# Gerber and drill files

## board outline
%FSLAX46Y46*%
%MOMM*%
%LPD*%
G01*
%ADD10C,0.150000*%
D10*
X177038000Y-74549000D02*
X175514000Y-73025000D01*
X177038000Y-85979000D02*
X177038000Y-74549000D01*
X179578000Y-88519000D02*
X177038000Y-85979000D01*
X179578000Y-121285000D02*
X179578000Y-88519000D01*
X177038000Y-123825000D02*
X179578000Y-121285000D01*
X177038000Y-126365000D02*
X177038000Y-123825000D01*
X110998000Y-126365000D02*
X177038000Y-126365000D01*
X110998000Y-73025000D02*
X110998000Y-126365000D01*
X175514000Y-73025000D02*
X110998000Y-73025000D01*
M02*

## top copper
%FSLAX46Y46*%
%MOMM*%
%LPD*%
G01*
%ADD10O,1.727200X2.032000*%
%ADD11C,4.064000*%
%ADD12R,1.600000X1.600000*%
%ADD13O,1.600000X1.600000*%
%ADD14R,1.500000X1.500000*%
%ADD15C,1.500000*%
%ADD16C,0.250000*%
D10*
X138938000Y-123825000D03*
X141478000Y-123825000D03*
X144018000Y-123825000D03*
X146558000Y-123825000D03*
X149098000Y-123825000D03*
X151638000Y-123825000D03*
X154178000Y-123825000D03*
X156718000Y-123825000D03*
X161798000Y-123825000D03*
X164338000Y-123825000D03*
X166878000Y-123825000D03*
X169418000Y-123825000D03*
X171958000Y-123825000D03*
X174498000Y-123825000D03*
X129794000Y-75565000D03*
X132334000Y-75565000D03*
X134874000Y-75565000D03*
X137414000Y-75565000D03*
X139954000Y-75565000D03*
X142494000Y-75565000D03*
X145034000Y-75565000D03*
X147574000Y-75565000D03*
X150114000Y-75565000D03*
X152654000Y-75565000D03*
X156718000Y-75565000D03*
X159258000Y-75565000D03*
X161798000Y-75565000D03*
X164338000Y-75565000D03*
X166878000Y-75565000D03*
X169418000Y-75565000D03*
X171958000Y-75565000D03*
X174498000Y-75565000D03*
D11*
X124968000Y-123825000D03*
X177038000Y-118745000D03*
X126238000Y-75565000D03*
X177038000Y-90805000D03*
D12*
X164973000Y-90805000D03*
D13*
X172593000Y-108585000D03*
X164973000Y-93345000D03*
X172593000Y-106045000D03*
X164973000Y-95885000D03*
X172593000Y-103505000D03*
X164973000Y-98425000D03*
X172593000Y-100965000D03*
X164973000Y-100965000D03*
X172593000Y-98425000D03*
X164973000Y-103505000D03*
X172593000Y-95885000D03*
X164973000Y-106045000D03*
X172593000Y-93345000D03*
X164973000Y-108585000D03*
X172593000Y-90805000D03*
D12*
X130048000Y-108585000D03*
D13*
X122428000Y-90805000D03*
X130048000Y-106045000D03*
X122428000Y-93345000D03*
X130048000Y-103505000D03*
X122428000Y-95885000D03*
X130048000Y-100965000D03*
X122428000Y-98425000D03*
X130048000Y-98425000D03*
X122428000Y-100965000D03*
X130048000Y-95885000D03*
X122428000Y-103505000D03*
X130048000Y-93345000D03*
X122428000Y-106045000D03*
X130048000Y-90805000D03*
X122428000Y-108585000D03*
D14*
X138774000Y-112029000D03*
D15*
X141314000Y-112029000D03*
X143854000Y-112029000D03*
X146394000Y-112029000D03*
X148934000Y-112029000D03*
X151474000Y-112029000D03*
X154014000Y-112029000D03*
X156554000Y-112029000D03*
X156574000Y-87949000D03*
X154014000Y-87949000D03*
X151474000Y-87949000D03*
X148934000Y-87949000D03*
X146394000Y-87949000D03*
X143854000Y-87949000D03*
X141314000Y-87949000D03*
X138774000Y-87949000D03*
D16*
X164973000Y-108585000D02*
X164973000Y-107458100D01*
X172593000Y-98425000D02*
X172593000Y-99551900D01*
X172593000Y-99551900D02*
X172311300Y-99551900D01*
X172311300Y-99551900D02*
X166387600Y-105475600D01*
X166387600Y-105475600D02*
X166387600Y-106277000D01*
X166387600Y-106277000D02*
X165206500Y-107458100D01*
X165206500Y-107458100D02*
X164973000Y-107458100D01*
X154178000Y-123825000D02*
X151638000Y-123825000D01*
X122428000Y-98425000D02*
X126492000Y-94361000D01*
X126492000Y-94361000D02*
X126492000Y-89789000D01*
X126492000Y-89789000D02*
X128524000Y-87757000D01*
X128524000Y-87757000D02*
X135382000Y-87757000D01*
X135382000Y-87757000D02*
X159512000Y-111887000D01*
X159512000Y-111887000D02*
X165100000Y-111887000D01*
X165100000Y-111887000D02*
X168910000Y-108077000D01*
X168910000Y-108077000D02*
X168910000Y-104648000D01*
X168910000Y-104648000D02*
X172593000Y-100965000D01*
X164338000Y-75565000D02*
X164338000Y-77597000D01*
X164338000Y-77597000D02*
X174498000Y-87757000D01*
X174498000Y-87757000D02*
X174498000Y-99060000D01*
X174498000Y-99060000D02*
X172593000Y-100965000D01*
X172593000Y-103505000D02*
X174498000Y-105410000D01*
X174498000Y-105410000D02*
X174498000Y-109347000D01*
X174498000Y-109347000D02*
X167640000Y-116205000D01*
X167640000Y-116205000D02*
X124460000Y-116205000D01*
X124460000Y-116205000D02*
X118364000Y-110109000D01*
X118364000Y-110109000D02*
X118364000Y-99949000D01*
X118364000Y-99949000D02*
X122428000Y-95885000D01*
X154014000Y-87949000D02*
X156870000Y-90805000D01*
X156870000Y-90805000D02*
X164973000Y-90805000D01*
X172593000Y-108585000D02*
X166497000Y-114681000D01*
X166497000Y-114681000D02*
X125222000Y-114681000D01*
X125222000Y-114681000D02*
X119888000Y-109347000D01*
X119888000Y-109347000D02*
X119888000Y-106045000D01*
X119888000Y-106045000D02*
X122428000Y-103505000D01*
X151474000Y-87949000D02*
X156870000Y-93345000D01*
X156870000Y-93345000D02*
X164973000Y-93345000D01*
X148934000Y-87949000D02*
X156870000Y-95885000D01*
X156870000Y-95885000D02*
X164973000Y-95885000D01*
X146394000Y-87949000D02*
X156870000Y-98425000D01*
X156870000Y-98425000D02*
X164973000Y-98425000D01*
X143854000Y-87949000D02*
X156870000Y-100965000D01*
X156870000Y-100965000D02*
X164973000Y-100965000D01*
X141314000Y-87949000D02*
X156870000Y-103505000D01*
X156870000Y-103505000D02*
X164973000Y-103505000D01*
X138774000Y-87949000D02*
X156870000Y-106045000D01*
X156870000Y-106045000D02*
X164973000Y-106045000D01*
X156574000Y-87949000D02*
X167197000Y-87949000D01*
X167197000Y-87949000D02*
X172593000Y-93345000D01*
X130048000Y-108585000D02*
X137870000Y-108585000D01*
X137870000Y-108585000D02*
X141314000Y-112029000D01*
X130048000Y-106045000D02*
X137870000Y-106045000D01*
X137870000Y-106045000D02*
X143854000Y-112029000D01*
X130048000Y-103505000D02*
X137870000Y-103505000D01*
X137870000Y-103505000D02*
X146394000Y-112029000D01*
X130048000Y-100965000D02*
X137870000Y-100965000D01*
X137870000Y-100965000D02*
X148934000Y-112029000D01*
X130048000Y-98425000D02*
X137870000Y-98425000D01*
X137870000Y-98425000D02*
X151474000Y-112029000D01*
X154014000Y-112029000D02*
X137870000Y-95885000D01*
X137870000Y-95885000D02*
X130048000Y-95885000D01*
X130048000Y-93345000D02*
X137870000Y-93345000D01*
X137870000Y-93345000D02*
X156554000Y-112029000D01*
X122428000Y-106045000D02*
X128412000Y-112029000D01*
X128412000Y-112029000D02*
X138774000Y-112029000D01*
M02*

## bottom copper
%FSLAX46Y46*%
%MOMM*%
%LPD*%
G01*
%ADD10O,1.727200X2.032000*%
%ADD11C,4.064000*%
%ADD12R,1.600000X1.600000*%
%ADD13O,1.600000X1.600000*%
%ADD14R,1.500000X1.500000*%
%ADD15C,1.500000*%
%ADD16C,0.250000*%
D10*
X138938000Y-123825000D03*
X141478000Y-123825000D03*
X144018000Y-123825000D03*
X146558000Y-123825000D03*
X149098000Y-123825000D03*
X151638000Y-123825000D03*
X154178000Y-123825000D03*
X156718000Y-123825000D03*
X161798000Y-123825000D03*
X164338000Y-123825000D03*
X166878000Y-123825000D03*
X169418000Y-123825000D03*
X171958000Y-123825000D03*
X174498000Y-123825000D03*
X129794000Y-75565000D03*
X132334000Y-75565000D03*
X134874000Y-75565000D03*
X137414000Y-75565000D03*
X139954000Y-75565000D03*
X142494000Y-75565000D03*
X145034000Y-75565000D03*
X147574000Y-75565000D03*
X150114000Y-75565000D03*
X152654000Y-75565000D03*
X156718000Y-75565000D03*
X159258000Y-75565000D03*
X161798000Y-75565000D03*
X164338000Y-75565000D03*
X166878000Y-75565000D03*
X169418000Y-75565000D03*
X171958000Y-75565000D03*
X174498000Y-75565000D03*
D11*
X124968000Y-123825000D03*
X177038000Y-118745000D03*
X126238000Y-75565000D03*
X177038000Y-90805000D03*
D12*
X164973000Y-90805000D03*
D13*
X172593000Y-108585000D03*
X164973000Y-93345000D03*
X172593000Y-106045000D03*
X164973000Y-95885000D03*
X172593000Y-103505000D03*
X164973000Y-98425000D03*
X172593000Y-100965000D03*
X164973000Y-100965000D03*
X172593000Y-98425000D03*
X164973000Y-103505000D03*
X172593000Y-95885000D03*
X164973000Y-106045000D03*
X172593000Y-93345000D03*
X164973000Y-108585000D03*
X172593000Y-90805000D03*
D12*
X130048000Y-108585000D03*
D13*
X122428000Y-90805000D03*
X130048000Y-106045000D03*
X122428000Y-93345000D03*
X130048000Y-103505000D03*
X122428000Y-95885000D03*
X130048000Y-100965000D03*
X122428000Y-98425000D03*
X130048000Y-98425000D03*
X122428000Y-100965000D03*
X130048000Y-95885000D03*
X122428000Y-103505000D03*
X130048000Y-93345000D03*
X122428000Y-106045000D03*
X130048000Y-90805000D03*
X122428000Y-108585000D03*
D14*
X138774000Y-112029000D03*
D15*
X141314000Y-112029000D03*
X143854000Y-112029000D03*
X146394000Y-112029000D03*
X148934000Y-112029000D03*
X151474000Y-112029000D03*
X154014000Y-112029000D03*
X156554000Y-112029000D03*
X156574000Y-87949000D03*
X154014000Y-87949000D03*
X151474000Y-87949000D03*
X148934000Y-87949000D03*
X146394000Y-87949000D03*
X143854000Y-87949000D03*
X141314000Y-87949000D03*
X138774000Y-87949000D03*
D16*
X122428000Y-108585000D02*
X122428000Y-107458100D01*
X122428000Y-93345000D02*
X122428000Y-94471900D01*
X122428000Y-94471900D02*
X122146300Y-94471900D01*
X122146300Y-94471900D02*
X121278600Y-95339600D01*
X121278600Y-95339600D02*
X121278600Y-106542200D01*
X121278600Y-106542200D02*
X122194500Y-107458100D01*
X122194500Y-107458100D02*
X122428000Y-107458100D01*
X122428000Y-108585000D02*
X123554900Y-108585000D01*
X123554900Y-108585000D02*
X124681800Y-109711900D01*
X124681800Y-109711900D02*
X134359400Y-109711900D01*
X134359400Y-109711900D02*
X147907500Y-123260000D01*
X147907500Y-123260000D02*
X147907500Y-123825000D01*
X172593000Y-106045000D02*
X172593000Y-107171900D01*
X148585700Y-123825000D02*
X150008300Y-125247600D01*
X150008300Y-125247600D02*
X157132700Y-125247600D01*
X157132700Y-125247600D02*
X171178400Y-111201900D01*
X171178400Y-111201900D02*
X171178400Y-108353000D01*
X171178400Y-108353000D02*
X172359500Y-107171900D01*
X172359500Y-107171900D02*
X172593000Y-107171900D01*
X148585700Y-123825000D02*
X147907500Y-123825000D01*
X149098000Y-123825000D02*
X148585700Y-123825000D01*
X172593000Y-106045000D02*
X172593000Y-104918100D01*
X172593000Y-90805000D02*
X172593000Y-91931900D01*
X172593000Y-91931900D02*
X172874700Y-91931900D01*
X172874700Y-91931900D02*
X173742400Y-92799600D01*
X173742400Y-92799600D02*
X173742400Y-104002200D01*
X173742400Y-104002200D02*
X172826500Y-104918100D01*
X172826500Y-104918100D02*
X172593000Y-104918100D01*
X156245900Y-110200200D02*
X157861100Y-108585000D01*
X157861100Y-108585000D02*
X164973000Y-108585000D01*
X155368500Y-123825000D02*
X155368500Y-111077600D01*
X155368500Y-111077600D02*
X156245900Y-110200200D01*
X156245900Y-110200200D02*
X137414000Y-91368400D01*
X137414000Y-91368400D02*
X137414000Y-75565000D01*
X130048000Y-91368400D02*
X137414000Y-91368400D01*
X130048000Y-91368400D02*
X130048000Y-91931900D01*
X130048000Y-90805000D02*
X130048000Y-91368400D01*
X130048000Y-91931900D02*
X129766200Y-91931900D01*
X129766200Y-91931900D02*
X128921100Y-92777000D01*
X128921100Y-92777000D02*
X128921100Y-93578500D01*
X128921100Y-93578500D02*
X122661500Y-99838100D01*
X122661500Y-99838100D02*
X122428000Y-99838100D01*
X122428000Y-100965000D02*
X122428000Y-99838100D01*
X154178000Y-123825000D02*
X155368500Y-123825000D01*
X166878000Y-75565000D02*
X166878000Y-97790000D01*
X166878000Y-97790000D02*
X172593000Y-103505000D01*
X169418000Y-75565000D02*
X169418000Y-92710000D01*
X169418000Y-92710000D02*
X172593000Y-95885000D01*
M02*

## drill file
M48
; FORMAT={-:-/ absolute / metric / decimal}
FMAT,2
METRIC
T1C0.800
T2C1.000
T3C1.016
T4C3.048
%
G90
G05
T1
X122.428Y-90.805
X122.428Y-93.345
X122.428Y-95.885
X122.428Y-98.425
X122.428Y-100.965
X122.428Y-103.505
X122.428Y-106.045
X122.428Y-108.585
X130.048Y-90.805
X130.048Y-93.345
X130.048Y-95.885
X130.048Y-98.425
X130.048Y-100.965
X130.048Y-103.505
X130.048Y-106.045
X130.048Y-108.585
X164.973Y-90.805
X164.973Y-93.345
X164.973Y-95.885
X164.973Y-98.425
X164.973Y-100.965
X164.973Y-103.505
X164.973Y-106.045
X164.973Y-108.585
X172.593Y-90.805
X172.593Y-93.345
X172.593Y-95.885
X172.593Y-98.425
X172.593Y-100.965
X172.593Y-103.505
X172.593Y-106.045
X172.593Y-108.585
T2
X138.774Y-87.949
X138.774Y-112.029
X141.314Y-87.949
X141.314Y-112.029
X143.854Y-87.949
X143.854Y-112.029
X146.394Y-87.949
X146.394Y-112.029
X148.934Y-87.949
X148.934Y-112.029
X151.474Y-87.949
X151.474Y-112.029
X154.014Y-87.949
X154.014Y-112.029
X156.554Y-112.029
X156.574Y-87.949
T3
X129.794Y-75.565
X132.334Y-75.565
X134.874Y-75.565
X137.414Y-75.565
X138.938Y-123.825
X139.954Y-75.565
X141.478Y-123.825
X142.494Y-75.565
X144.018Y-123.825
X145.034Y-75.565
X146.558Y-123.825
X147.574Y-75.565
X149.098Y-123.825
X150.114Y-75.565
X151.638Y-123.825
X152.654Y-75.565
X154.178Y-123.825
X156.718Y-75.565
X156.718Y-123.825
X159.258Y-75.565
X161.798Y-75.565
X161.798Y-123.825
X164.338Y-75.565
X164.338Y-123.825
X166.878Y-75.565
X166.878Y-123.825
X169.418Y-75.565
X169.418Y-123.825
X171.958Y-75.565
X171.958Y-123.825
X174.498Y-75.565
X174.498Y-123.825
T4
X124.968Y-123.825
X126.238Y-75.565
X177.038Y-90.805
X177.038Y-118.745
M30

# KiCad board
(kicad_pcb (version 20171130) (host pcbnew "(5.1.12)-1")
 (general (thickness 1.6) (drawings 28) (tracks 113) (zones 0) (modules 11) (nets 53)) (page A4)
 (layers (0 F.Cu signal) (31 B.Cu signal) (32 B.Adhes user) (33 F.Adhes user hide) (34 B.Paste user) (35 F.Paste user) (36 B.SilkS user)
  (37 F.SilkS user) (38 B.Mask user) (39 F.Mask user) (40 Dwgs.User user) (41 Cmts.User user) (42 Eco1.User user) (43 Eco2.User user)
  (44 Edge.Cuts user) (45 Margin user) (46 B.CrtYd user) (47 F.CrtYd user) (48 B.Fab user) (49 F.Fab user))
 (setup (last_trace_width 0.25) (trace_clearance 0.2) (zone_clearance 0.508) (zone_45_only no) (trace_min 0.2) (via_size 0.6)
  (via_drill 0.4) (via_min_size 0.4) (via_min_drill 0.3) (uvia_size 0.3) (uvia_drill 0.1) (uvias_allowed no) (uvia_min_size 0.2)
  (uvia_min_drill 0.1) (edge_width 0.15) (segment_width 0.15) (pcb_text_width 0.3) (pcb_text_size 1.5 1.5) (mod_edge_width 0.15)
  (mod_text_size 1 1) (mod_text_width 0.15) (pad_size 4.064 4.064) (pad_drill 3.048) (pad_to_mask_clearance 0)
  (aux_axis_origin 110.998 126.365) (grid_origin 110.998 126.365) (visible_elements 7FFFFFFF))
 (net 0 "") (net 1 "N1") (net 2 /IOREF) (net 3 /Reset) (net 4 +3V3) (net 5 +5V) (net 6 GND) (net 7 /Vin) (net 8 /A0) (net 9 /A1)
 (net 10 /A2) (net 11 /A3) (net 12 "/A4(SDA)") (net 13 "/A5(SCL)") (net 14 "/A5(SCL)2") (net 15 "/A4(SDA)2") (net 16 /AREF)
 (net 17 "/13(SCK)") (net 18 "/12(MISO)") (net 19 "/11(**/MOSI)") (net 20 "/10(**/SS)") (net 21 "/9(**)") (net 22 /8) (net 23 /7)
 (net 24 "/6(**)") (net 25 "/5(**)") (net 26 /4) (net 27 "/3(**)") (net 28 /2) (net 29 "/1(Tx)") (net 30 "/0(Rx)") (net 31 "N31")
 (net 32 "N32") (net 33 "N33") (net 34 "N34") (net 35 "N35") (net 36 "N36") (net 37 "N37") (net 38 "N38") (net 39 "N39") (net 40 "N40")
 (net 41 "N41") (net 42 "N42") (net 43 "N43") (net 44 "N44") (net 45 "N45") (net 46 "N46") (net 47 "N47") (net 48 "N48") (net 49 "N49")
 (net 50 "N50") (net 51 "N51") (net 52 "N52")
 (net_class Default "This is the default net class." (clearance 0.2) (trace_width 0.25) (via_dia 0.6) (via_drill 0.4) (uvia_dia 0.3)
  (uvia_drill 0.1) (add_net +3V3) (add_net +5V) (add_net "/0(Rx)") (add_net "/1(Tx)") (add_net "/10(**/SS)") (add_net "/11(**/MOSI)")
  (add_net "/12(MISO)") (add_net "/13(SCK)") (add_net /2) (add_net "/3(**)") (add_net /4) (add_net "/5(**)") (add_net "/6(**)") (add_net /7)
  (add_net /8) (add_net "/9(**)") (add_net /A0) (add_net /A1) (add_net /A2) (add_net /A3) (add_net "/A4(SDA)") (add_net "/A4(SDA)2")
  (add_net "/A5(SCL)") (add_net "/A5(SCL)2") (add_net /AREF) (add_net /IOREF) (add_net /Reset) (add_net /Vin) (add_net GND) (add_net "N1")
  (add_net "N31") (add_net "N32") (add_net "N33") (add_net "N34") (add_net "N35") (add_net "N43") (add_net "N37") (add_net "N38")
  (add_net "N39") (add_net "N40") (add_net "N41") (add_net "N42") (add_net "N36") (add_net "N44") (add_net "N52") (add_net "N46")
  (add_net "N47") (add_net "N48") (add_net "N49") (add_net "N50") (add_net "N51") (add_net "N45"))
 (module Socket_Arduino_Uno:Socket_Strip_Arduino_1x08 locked (layer F.Cu) (at 138.938 123.825)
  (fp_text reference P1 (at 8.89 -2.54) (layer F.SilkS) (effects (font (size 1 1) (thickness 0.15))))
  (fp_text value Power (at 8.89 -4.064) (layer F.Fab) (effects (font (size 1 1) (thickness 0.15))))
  (pad 1 thru_hole oval (at 0 0) (size 1.7272 2.032) (drill 1.016) (layers *.Cu *.Mask F.SilkS) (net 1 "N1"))
  (pad 2 thru_hole oval (at 2.54 0) (size 1.7272 2.032) (drill 1.016) (layers *.Cu *.Mask F.SilkS) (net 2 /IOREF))
  (pad 3 thru_hole oval (at 5.08 0) (size 1.7272 2.032) (drill 1.016) (layers *.Cu *.Mask F.SilkS) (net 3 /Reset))
  (pad 4 thru_hole oval (at 7.62 0) (size 1.7272 2.032) (drill 1.016) (layers *.Cu *.Mask F.SilkS) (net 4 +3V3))
  (pad 5 thru_hole oval (at 10.16 0) (size 1.7272 2.032) (drill 1.016) (layers *.Cu *.Mask F.SilkS) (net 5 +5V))
  (pad 6 thru_hole oval (at 12.7 0) (size 1.7272 2.032) (drill 1.016) (layers *.Cu *.Mask F.SilkS) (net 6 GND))
  (pad 7 thru_hole oval (at 15.24 0) (size 1.7272 2.032) (drill 1.016) (layers *.Cu *.Mask F.SilkS) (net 6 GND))
  (pad 8 thru_hole oval (at 17.78 0) (size 1.7272 2.032) (drill 1.016) (layers *.Cu *.Mask F.SilkS) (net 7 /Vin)))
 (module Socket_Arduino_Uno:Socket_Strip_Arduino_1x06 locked (layer F.Cu) (at 161.798 123.825)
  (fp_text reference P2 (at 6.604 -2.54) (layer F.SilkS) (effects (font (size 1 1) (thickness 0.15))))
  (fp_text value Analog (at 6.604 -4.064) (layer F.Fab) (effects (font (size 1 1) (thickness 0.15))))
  (pad 1 thru_hole oval (at 0 0) (size 1.7272 2.032) (drill 1.016) (layers *.Cu *.Mask F.SilkS) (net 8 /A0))
  (pad 2 thru_hole oval (at 2.54 0) (size 1.7272 2.032) (drill 1.016) (layers *.Cu *.Mask F.SilkS) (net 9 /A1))
  (pad 3 thru_hole oval (at 5.08 0) (size 1.7272 2.032) (drill 1.016) (layers *.Cu *.Mask F.SilkS) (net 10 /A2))
  (pad 4 thru_hole oval (at 7.62 0) (size 1.7272 2.032) (drill 1.016) (layers *.Cu *.Mask F.SilkS) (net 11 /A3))
  (pad 5 thru_hole oval (at 10.16 0) (size 1.7272 2.032) (drill 1.016) (layers *.Cu *.Mask F.SilkS) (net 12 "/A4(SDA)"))
  (pad 6 thru_hole oval (at 12.7 0) (size 1.7272 2.032) (drill 1.016) (layers *.Cu *.Mask F.SilkS) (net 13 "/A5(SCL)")))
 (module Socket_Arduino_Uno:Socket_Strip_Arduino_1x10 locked (layer F.Cu) (at 129.794 75.565)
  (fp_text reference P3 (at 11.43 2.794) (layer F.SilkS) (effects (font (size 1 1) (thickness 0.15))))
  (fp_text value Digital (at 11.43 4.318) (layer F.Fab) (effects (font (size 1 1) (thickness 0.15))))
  (pad 1 thru_hole oval (at 0 0) (size 1.7272 2.032) (drill 1.016) (layers *.Cu *.Mask F.SilkS) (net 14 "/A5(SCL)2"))
  (pad 2 thru_hole oval (at 2.54 0) (size 1.7272 2.032) (drill 1.016) (layers *.Cu *.Mask F.SilkS) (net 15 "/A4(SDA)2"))
  (pad 3 thru_hole oval (at 5.08 0) (size 1.7272 2.032) (drill 1.016) (layers *.Cu *.Mask F.SilkS) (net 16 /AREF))
  (pad 4 thru_hole oval (at 7.62 0) (size 1.7272 2.032) (drill 1.016) (layers *.Cu *.Mask F.SilkS) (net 6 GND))
  (pad 5 thru_hole oval (at 10.16 0) (size 1.7272 2.032) (drill 1.016) (layers *.Cu *.Mask F.SilkS) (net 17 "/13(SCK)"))
  (pad 6 thru_hole oval (at 12.7 0) (size 1.7272 2.032) (drill 1.016) (layers *.Cu *.Mask F.SilkS) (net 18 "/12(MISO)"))
  (pad 7 thru_hole oval (at 15.24 0) (size 1.7272 2.032) (drill 1.016) (layers *.Cu *.Mask F.SilkS) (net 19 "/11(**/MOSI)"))
  (pad 8 thru_hole oval (at 17.78 0) (size 1.7272 2.032) (drill 1.016) (layers *.Cu *.Mask F.SilkS) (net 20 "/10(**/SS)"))
  (pad 9 thru_hole oval (at 20.32 0) (size 1.7272 2.032) (drill 1.016) (layers *.Cu *.Mask F.SilkS) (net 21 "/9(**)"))
  (pad 10 thru_hole oval (at 22.86 0) (size 1.7272 2.032) (drill 1.016) (layers *.Cu *.Mask F.SilkS) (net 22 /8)))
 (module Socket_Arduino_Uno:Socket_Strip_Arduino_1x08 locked (layer F.Cu) (at 156.718 75.565)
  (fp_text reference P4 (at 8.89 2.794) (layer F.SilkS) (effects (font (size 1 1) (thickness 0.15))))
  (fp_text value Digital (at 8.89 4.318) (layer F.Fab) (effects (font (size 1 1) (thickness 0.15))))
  (pad 1 thru_hole oval (at 0 0) (size 1.7272 2.032) (drill 1.016) (layers *.Cu *.Mask F.SilkS) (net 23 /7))
  (pad 2 thru_hole oval (at 2.54 0) (size 1.7272 2.032) (drill 1.016) (layers *.Cu *.Mask F.SilkS) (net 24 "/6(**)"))
  (pad 3 thru_hole oval (at 5.08 0) (size 1.7272 2.032) (drill 1.016) (layers *.Cu *.Mask F.SilkS) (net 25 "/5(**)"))
  (pad 4 thru_hole oval (at 7.62 0) (size 1.7272 2.032) (drill 1.016) (layers *.Cu *.Mask F.SilkS) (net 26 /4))
  (pad 5 thru_hole oval (at 10.16 0) (size 1.7272 2.032) (drill 1.016) (layers *.Cu *.Mask F.SilkS) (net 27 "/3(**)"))
  (pad 6 thru_hole oval (at 12.7 0) (size 1.7272 2.032) (drill 1.016) (layers *.Cu *.Mask F.SilkS) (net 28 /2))
  (pad 7 thru_hole oval (at 15.24 0) (size 1.7272 2.032) (drill 1.016) (layers *.Cu *.Mask F.SilkS) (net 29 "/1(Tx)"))
  (pad 8 thru_hole oval (at 17.78 0) (size 1.7272 2.032) (drill 1.016) (layers *.Cu *.Mask F.SilkS) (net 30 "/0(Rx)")))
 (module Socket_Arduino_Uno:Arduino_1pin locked (layer F.Cu) (at 124.968 123.825)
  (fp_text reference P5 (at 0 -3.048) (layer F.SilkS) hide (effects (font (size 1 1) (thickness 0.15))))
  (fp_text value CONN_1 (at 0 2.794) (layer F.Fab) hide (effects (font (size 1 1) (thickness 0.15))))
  (pad 1 thru_hole circle (at 0 0) (size 4.064 4.064) (drill 3.048) (layers *.Cu *.Mask F.SilkS) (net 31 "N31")))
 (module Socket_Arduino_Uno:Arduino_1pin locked (layer F.Cu) (at 177.038 118.745)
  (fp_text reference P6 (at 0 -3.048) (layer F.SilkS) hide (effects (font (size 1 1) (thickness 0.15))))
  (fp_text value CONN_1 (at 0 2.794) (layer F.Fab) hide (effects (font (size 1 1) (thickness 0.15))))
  (pad 1 thru_hole circle (at 0 0) (size 4.064 4.064) (drill 3.048) (layers *.Cu *.Mask F.SilkS) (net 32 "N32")))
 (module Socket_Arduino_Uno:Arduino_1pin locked (layer F.Cu) (at 126.238 75.565)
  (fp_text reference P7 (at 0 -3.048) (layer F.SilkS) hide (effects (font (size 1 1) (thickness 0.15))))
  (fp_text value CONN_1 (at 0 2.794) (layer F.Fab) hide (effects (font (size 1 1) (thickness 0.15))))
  (pad 1 thru_hole circle (at 0 0) (size 4.064 4.064) (drill 3.048) (layers *.Cu *.Mask F.SilkS) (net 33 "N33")))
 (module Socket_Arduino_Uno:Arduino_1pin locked (layer F.Cu) (at 177.038 90.805)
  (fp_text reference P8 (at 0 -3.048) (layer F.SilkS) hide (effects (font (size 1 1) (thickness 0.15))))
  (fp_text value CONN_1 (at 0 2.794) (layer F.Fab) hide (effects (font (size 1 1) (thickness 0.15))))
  (pad 1 thru_hole circle (at 0 0) (size 4.064 4.064) (drill 3.048) (layers *.Cu *.Mask F.SilkS) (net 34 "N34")))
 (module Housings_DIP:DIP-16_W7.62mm (layer F.Cu) (at 164.973 90.805)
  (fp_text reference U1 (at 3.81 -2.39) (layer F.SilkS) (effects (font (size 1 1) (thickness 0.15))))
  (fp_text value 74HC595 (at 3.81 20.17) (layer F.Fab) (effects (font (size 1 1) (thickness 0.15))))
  (pad 1 thru_hole rect (at 0 0) (size 1.6 1.6) (drill 0.8) (layers *.Cu *.Mask) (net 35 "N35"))
  (pad 9 thru_hole oval (at 7.62 17.78) (size 1.6 1.6) (drill 0.8) (layers *.Cu *.Mask) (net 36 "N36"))
  (pad 2 thru_hole oval (at 0 2.54) (size 1.6 1.6) (drill 0.8) (layers *.Cu *.Mask) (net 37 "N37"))
  (pad 10 thru_hole oval (at 7.62 15.24) (size 1.6 1.6) (drill 0.8) (layers *.Cu *.Mask) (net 5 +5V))
  (pad 3 thru_hole oval (at 0 5.08) (size 1.6 1.6) (drill 0.8) (layers *.Cu *.Mask) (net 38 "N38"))
  (pad 11 thru_hole oval (at 7.62 12.7) (size 1.6 1.6) (drill 0.8) (layers *.Cu *.Mask) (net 27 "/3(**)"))
  (pad 4 thru_hole oval (at 0 7.62) (size 1.6 1.6) (drill 0.8) (layers *.Cu *.Mask) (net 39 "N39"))
  (pad 12 thru_hole oval (at 7.62 10.16) (size 1.6 1.6) (drill 0.8) (layers *.Cu *.Mask) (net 26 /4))
  (pad 5 thru_hole oval (at 0 10.16) (size 1.6 1.6) (drill 0.8) (layers *.Cu *.Mask) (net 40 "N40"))
  (pad 13 thru_hole oval (at 7.62 7.62) (size 1.6 1.6) (drill 0.8) (layers *.Cu *.Mask) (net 6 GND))
  (pad 6 thru_hole oval (at 0 12.7) (size 1.6 1.6) (drill 0.8) (layers *.Cu *.Mask) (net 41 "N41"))
  (pad 14 thru_hole oval (at 7.62 5.08) (size 1.6 1.6) (drill 0.8) (layers *.Cu *.Mask) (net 28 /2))
  (pad 7 thru_hole oval (at 0 15.24) (size 1.6 1.6) (drill 0.8) (layers *.Cu *.Mask) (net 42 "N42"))
  (pad 15 thru_hole oval (at 7.62 2.54) (size 1.6 1.6) (drill 0.8) (layers *.Cu *.Mask) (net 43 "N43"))
  (pad 8 thru_hole oval (at 0 17.78) (size 1.6 1.6) (drill 0.8) (layers *.Cu *.Mask) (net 6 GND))
  (pad 16 thru_hole oval (at 7.62 0) (size 1.6 1.6) (drill 0.8) (layers *.Cu *.Mask) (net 5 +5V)))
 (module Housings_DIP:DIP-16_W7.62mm (layer F.Cu) (at 130.048 108.585 180)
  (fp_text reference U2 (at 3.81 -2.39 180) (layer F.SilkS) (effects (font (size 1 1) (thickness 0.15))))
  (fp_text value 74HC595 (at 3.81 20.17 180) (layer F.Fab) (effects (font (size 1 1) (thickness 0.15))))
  (pad 1 thru_hole rect (at 0 0 180) (size 1.6 1.6) (drill 0.8) (layers *.Cu *.Mask) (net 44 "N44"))
  (pad 9 thru_hole oval (at 7.62 17.78 180) (size 1.6 1.6) (drill 0.8) (layers *.Cu *.Mask) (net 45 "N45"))
  (pad 2 thru_hole oval (at 0 2.54 180) (size 1.6 1.6) (drill 0.8) (layers *.Cu *.Mask) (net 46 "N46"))
  (pad 10 thru_hole oval (at 7.62 15.24 180) (size 1.6 1.6) (drill 0.8) (layers *.Cu *.Mask) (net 5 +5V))
  (pad 3 thru_hole oval (at 0 5.08 180) (size 1.6 1.6) (drill 0.8) (layers *.Cu *.Mask) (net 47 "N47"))
  (pad 11 thru_hole oval (at 7.62 12.7 180) (size 1.6 1.6) (drill 0.8) (layers *.Cu *.Mask) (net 27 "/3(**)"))
  (pad 4 thru_hole oval (at 0 7.62 180) (size 1.6 1.6) (drill 0.8) (layers *.Cu *.Mask) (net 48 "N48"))
  (pad 12 thru_hole oval (at 7.62 10.16 180) (size 1.6 1.6) (drill 0.8) (layers *.Cu *.Mask) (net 26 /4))
  (pad 5 thru_hole oval (at 0 10.16 180) (size 1.6 1.6) (drill 0.8) (layers *.Cu *.Mask) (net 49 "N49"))
  (pad 13 thru_hole oval (at 7.62 7.62 180) (size 1.6 1.6) (drill 0.8) (layers *.Cu *.Mask) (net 6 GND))
  (pad 6 thru_hole oval (at 0 12.7 180) (size 1.6 1.6) (drill 0.8) (layers *.Cu *.Mask) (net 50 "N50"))
  (pad 14 thru_hole oval (at 7.62 5.08 180) (size 1.6 1.6) (drill 0.8) (layers *.Cu *.Mask) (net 36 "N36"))
  (pad 7 thru_hole oval (at 0 15.24 180) (size 1.6 1.6) (drill 0.8) (layers *.Cu *.Mask) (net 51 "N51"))
  (pad 15 thru_hole oval (at 7.62 2.54 180) (size 1.6 1.6) (drill 0.8) (layers *.Cu *.Mask) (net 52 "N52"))
  (pad 8 thru_hole oval (at 0 17.78 180) (size 1.6 1.6) (drill 0.8) (layers *.Cu *.Mask) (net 6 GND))
  (pad 16 thru_hole oval (at 7.62 0 180) (size 1.6 1.6) (drill 0.8) (layers *.Cu *.Mask) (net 5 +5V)))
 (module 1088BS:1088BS (layer F.Cu) (at 147.574 99.949)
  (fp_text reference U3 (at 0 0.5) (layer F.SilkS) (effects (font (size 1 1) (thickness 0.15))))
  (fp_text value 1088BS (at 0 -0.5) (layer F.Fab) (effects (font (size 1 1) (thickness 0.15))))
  (pad 1 thru_hole rect (at -8.8 12.08) (size 1.5 1.5) (drill 1) (layers *.Cu *.Mask F.SilkS) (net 52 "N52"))
  (pad 2 thru_hole circle (at -6.26 12.08) (size 1.5 1.5) (drill 1) (layers *.Cu *.Mask F.SilkS) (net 44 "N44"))
  (pad 3 thru_hole circle (at -3.72 12.08) (size 1.5 1.5) (drill 1) (layers *.Cu *.Mask F.SilkS) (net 46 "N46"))
  (pad 4 thru_hole circle (at -1.18 12.08) (size 1.5 1.5) (drill 1) (layers *.Cu *.Mask F.SilkS) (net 47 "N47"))
  (pad 5 thru_hole circle (at 1.36 12.08) (size 1.5 1.5) (drill 1) (layers *.Cu *.Mask F.SilkS) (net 48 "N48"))
  (pad 6 thru_hole circle (at 3.9 12.08) (size 1.5 1.5) (drill 1) (layers *.Cu *.Mask F.SilkS) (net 49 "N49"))
  (pad 7 thru_hole circle (at 6.44 12.08) (size 1.5 1.5) (drill 1) (layers *.Cu *.Mask F.SilkS) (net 50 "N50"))
  (pad 8 thru_hole circle (at 8.98 12.08) (size 1.5 1.5) (drill 1) (layers *.Cu *.Mask F.SilkS) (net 51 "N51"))
  (pad 9 thru_hole circle (at 9 -12) (size 1.5 1.5) (drill 1) (layers *.Cu *.Mask F.SilkS) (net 43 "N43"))
  (pad 10 thru_hole circle (at 6.44 -12) (size 1.5 1.5) (drill 1) (layers *.Cu *.Mask F.SilkS) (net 35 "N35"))
  (pad 11 thru_hole circle (at 3.9 -12) (size 1.5 1.5) (drill 1) (layers *.Cu *.Mask F.SilkS) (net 37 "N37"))
  (pad 12 thru_hole circle (at 1.36 -12) (size 1.5 1.5) (drill 1) (layers *.Cu *.Mask F.SilkS) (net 38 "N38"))
  (pad 13 thru_hole circle (at -1.18 -12) (size 1.5 1.5) (drill 1) (layers *.Cu *.Mask F.SilkS) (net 39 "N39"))
  (pad 14 thru_hole circle (at -3.72 -12) (size 1.5 1.5) (drill 1) (layers *.Cu *.Mask F.SilkS) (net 40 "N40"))
  (pad 15 thru_hole circle (at -6.26 -12) (size 1.5 1.5) (drill 1) (layers *.Cu *.Mask F.SilkS) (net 41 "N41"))
  (pad 16 thru_hole circle (at -8.8 -12) (size 1.5 1.5) (drill 1) (layers *.Cu *.Mask F.SilkS) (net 42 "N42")))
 (gr_line (start 177.038 74.549) (end 175.514 73.025) (angle 90) (layer Edge.Cuts) (width 0.15))
 (gr_line (start 177.038 85.979) (end 177.038 74.549) (angle 90) (layer Edge.Cuts) (width 0.15))
 (gr_line (start 179.578 88.519) (end 177.038 85.979) (angle 90) (layer Edge.Cuts) (width 0.15))
 (gr_line (start 179.578 121.285) (end 179.578 88.519) (angle 90) (layer Edge.Cuts) (width 0.15))
 (gr_line (start 177.038 123.825) (end 179.578 121.285) (angle 90) (layer Edge.Cuts) (width 0.15))
 (gr_line (start 177.038 126.365) (end 177.038 123.825) (angle 90) (layer Edge.Cuts) (width 0.15))
 (gr_line (start 110.998 126.365) (end 177.038 126.365) (angle 90) (layer Edge.Cuts) (width 0.15))
 (gr_line (start 110.998 73.025) (end 110.998 126.365) (angle 90) (layer Edge.Cuts) (width 0.15))
 (gr_line (start 175.514 73.025) (end 110.998 73.025) (angle 90) (layer Edge.Cuts) (width 0.15))
 (segment (start 122.428 108.585) (end 122.428 107.4581) (width 0.25) (layer B.Cu) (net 5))
 (segment (start 122.428 93.345) (end 122.428 94.4719) (width 0.25) (layer B.Cu) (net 5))
 (segment (start 122.428 94.4719) (end 122.1463 94.4719) (width 0.25) (layer B.Cu) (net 5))
 (segment (start 122.1463 94.4719) (end 121.2786 95.3396) (width 0.25) (layer B.Cu) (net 5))
 (segment (start 121.2786 95.3396) (end 121.2786 106.5422) (width 0.25) (layer B.Cu) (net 5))
 (segment (start 121.2786 106.5422) (end 122.1945 107.4581) (width 0.25) (layer B.Cu) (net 5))
 (segment (start 122.1945 107.4581) (end 122.428 107.4581) (width 0.25) (layer B.Cu) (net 5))
 (segment (start 122.428 108.585) (end 123.5549 108.585) (width 0.25) (layer B.Cu) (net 5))
 (segment (start 123.5549 108.585) (end 124.6818 109.7119) (width 0.25) (layer B.Cu) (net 5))
 (segment (start 124.6818 109.7119) (end 134.3594 109.7119) (width 0.25) (layer B.Cu) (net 5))
 (segment (start 134.3594 109.7119) (end 147.9075 123.26) (width 0.25) (layer B.Cu) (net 5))
 (segment (start 147.9075 123.26) (end 147.9075 123.825) (width 0.25) (layer B.Cu) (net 5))
 (segment (start 172.593 106.045) (end 172.593 107.1719) (width 0.25) (layer B.Cu) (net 5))
 (segment (start 148.5857 123.825) (end 150.0083 125.2476) (width 0.25) (layer B.Cu) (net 5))
 (segment (start 150.0083 125.2476) (end 157.1327 125.2476) (width 0.25) (layer B.Cu) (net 5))
 (segment (start 157.1327 125.2476) (end 171.1784 111.2019) (width 0.25) (layer B.Cu) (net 5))
 (segment (start 171.1784 111.2019) (end 171.1784 108.353) (width 0.25) (layer B.Cu) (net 5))
 (segment (start 171.1784 108.353) (end 172.3595 107.1719) (width 0.25) (layer B.Cu) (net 5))
 (segment (start 172.3595 107.1719) (end 172.593 107.1719) (width 0.25) (layer B.Cu) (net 5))
 (segment (start 148.5857 123.825) (end 147.9075 123.825) (width 0.25) (layer B.Cu) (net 5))
 (segment (start 149.098 123.825) (end 148.5857 123.825) (width 0.25) (layer B.Cu) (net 5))
 (segment (start 172.593 106.045) (end 172.593 104.9181) (width 0.25) (layer B.Cu) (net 5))
 (segment (start 172.593 90.805) (end 172.593 91.9319) (width 0.25) (layer B.Cu) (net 5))
 (segment (start 172.593 91.9319) (end 172.8747 91.9319) (width 0.25) (layer B.Cu) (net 5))
 (segment (start 172.8747 91.9319) (end 173.7424 92.7996) (width 0.25) (layer B.Cu) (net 5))
 (segment (start 173.7424 92.7996) (end 173.7424 104.0022) (width 0.25) (layer B.Cu) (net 5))
 (segment (start 173.7424 104.0022) (end 172.8265 104.9181) (width 0.25) (layer B.Cu) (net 5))
 (segment (start 172.8265 104.9181) (end 172.593 104.9181) (width 0.25) (layer B.Cu) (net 5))
 (segment (start 164.973 108.585) (end 164.973 107.4581) (width 0.25) (layer F.Cu) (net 6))
 (segment (start 172.593 98.425) (end 172.593 99.5519) (width 0.25) (layer F.Cu) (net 6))
 (segment (start 172.593 99.5519) (end 172.3113 99.5519) (width 0.25) (layer F.Cu) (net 6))
 (segment (start 172.3113 99.5519) (end 166.3876 105.4756) (width 0.25) (layer F.Cu) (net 6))
 (segment (start 166.3876 105.4756) (end 166.3876 106.277) (width 0.25) (layer F.Cu) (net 6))
 (segment (start 166.3876 106.277) (end 165.2065 107.4581) (width 0.25) (layer F.Cu) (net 6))
 (segment (start 165.2065 107.4581) (end 164.973 107.4581) (width 0.25) (layer F.Cu) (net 6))
 (segment (start 156.2459 110.2002) (end 157.8611 108.585) (width 0.25) (layer B.Cu) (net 6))
 (segment (start 157.8611 108.585) (end 164.973 108.585) (width 0.25) (layer B.Cu) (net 6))
 (segment (start 155.3685 123.825) (end 155.3685 111.0776) (width 0.25) (layer B.Cu) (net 6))
 (segment (start 155.3685 111.0776) (end 156.2459 110.2002) (width 0.25) (layer B.Cu) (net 6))
 (segment (start 156.2459 110.2002) (end 137.414 91.3684) (width 0.25) (layer B.Cu) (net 6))
 (segment (start 137.414 91.3684) (end 137.414 75.565) (width 0.25) (layer B.Cu) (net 6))
 (segment (start 130.048 91.3684) (end 137.414 91.3684) (width 0.25) (layer B.Cu) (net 6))
 (segment (start 130.048 91.3684) (end 130.048 91.9319) (width 0.25) (layer B.Cu) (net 6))
 (segment (start 130.048 90.805) (end 130.048 91.3684) (width 0.25) (layer B.Cu) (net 6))
 (segment (start 130.048 91.9319) (end 129.7662 91.9319) (width 0.25) (layer B.Cu) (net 6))
 (segment (start 129.7662 91.9319) (end 128.9211 92.777) (width 0.25) (layer B.Cu) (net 6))
 (segment (start 128.9211 92.777) (end 128.9211 93.5785) (width 0.25) (layer B.Cu) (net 6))
 (segment (start 128.9211 93.5785) (end 122.6615 99.8381) (width 0.25) (layer B.Cu) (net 6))
 (segment (start 122.6615 99.8381) (end 122.428 99.8381) (width 0.25) (layer B.Cu) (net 6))
 (segment (start 122.428 100.965) (end 122.428 99.8381) (width 0.25) (layer B.Cu) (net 6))
 (segment (start 154.178 123.825) (end 155.3685 123.825) (width 0.25) (layer B.Cu) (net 6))
 (segment (start 154.178 123.825) (end 151.638 123.825) (width 0.25) (layer F.Cu) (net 6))
 (segment (start 122.428 98.425) (end 126.492 94.361) (width 0.25) (layer F.Cu) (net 26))
 (segment (start 126.492 94.361) (end 126.492 89.789) (width 0.25) (layer F.Cu) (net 26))
 (segment (start 126.492 89.789) (end 128.524 87.757) (width 0.25) (layer F.Cu) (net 26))
 (segment (start 128.524 87.757) (end 135.382 87.757) (width 0.25) (layer F.Cu) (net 26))
 (segment (start 135.382 87.757) (end 159.512 111.887) (width 0.25) (layer F.Cu) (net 26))
 (segment (start 159.512 111.887) (end 165.1 111.887) (width 0.25) (layer F.Cu) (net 26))
 (segment (start 165.1 111.887) (end 168.91 108.077) (width 0.25) (layer F.Cu) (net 26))
 (segment (start 168.91 108.077) (end 168.91 104.648) (width 0.25) (layer F.Cu) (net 26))
 (segment (start 168.91 104.648) (end 172.593 100.965) (width 0.25) (layer F.Cu) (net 26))
 (segment (start 164.338 75.565) (end 164.338 77.597) (width 0.25) (layer F.Cu) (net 26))
 (segment (start 164.338 77.597) (end 174.498 87.757) (width 0.25) (layer F.Cu) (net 26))
 (segment (start 174.498 87.757) (end 174.498 99.06) (width 0.25) (layer F.Cu) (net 26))
 (segment (start 174.498 99.06) (end 172.593 100.965) (width 0.25) (layer F.Cu) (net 26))
 (segment (start 172.593 103.505) (end 174.498 105.41) (width 0.25) (layer F.Cu) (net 27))
 (segment (start 174.498 105.41) (end 174.498 109.347) (width 0.25) (layer F.Cu) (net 27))
 (segment (start 174.498 109.347) (end 167.64 116.205) (width 0.25) (layer F.Cu) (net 27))
 (segment (start 167.64 116.205) (end 124.46 116.205) (width 0.25) (layer F.Cu) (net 27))
 (segment (start 124.46 116.205) (end 118.364 110.109) (width 0.25) (layer F.Cu) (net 27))
 (segment (start 118.364 110.109) (end 118.364 99.949) (width 0.25) (layer F.Cu) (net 27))
 (segment (start 118.364 99.949) (end 122.428 95.885) (width 0.25) (layer F.Cu) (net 27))
 (segment (start 166.878 75.565) (end 166.878 97.79) (width 0.25) (layer B.Cu) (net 27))
 (segment (start 166.878 97.79) (end 172.593 103.505) (width 0.25) (layer B.Cu) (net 27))
 (segment (start 169.418 75.565) (end 169.418 92.71) (width 0.25) (layer B.Cu) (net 28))
 (segment (start 169.418 92.71) (end 172.593 95.885) (width 0.25) (layer B.Cu) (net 28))
 (segment (start 154.014 87.949) (end 156.87 90.805) (width 0.25) (layer F.Cu) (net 35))
 (segment (start 156.87 90.805) (end 164.973 90.805) (width 0.25) (layer F.Cu) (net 35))
 (segment (start 172.593 108.585) (end 166.497 114.681) (width 0.25) (layer F.Cu) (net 36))
 (segment (start 166.497 114.681) (end 125.222 114.681) (width 0.25) (layer F.Cu) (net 36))
 (segment (start 125.222 114.681) (end 119.888 109.347) (width 0.25) (layer F.Cu) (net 36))
 (segment (start 119.888 109.347) (end 119.888 106.045) (width 0.25) (layer F.Cu) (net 36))
 (segment (start 119.888 106.045) (end 122.428 103.505) (width 0.25) (layer F.Cu) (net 36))
 (segment (start 151.474 87.949) (end 156.87 93.345) (width 0.25) (layer F.Cu) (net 37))
 (segment (start 156.87 93.345) (end 164.973 93.345) (width 0.25) (layer F.Cu) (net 37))
 (segment (start 148.934 87.949) (end 156.87 95.885) (width 0.25) (layer F.Cu) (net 38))
 (segment (start 156.87 95.885) (end 164.973 95.885) (width 0.25) (layer F.Cu) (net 38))
 (segment (start 146.394 87.949) (end 156.87 98.425) (width 0.25) (layer F.Cu) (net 39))
 (segment (start 156.87 98.425) (end 164.973 98.425) (width 0.25) (layer F.Cu) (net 39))
 (segment (start 143.854 87.949) (end 156.87 100.965) (width 0.25) (layer F.Cu) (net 40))
 (segment (start 156.87 100.965) (end 164.973 100.965) (width 0.25) (layer F.Cu) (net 40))
 (segment (start 141.314 87.949) (end 156.87 103.505) (width 0.25) (layer F.Cu) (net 41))
 (segment (start 156.87 103.505) (end 164.973 103.505) (width 0.25) (layer F.Cu) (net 41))
 (segment (start 138.774 87.949) (end 156.87 106.045) (width 0.25) (layer F.Cu) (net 42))
 (segment (start 156.87 106.045) (end 164.973 106.045) (width 0.25) (layer F.Cu) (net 42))
 (segment (start 156.574 87.949) (end 167.197 87.949) (width 0.25) (layer F.Cu) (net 43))
 (segment (start 167.197 87.949) (end 172.593 93.345) (width 0.25) (layer F.Cu) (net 43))
 (segment (start 130.048 108.585) (end 137.87 108.585) (width 0.25) (layer F.Cu) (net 44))
 (segment (start 137.87 108.585) (end 141.314 112.029) (width 0.25) (layer F.Cu) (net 44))
 (segment (start 130.048 106.045) (end 137.87 106.045) (width 0.25) (layer F.Cu) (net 46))
 (segment (start 137.87 106.045) (end 143.854 112.029) (width 0.25) (layer F.Cu) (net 46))
 (segment (start 130.048 103.505) (end 137.87 103.505) (width 0.25) (layer F.Cu) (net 47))
 (segment (start 137.87 103.505) (end 146.394 112.029) (width 0.25) (layer F.Cu) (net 47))
 (segment (start 130.048 100.965) (end 137.87 100.965) (width 0.25) (layer F.Cu) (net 48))
 (segment (start 137.87 100.965) (end 148.934 112.029) (width 0.25) (layer F.Cu) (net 48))
 (segment (start 130.048 98.425) (end 137.87 98.425) (width 0.25) (layer F.Cu) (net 49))
 (segment (start 137.87 98.425) (end 151.474 112.029) (width 0.25) (layer F.Cu) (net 49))
 (segment (start 154.014 112.029) (end 137.87 95.885) (width 0.25) (layer F.Cu) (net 50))
 (segment (start 137.87 95.885) (end 130.048 95.885) (width 0.25) (layer F.Cu) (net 50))
 (segment (start 130.048 93.345) (end 137.87 93.345) (width 0.25) (layer F.Cu) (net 51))
 (segment (start 137.87 93.345) (end 156.554 112.029) (width 0.25) (layer F.Cu) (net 51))
 (segment (start 122.428 106.045) (end 128.412 112.029) (width 0.25) (layer F.Cu) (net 52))
 (segment (start 128.412 112.029) (end 138.774 112.029) (width 0.25) (layer F.Cu) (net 52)))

